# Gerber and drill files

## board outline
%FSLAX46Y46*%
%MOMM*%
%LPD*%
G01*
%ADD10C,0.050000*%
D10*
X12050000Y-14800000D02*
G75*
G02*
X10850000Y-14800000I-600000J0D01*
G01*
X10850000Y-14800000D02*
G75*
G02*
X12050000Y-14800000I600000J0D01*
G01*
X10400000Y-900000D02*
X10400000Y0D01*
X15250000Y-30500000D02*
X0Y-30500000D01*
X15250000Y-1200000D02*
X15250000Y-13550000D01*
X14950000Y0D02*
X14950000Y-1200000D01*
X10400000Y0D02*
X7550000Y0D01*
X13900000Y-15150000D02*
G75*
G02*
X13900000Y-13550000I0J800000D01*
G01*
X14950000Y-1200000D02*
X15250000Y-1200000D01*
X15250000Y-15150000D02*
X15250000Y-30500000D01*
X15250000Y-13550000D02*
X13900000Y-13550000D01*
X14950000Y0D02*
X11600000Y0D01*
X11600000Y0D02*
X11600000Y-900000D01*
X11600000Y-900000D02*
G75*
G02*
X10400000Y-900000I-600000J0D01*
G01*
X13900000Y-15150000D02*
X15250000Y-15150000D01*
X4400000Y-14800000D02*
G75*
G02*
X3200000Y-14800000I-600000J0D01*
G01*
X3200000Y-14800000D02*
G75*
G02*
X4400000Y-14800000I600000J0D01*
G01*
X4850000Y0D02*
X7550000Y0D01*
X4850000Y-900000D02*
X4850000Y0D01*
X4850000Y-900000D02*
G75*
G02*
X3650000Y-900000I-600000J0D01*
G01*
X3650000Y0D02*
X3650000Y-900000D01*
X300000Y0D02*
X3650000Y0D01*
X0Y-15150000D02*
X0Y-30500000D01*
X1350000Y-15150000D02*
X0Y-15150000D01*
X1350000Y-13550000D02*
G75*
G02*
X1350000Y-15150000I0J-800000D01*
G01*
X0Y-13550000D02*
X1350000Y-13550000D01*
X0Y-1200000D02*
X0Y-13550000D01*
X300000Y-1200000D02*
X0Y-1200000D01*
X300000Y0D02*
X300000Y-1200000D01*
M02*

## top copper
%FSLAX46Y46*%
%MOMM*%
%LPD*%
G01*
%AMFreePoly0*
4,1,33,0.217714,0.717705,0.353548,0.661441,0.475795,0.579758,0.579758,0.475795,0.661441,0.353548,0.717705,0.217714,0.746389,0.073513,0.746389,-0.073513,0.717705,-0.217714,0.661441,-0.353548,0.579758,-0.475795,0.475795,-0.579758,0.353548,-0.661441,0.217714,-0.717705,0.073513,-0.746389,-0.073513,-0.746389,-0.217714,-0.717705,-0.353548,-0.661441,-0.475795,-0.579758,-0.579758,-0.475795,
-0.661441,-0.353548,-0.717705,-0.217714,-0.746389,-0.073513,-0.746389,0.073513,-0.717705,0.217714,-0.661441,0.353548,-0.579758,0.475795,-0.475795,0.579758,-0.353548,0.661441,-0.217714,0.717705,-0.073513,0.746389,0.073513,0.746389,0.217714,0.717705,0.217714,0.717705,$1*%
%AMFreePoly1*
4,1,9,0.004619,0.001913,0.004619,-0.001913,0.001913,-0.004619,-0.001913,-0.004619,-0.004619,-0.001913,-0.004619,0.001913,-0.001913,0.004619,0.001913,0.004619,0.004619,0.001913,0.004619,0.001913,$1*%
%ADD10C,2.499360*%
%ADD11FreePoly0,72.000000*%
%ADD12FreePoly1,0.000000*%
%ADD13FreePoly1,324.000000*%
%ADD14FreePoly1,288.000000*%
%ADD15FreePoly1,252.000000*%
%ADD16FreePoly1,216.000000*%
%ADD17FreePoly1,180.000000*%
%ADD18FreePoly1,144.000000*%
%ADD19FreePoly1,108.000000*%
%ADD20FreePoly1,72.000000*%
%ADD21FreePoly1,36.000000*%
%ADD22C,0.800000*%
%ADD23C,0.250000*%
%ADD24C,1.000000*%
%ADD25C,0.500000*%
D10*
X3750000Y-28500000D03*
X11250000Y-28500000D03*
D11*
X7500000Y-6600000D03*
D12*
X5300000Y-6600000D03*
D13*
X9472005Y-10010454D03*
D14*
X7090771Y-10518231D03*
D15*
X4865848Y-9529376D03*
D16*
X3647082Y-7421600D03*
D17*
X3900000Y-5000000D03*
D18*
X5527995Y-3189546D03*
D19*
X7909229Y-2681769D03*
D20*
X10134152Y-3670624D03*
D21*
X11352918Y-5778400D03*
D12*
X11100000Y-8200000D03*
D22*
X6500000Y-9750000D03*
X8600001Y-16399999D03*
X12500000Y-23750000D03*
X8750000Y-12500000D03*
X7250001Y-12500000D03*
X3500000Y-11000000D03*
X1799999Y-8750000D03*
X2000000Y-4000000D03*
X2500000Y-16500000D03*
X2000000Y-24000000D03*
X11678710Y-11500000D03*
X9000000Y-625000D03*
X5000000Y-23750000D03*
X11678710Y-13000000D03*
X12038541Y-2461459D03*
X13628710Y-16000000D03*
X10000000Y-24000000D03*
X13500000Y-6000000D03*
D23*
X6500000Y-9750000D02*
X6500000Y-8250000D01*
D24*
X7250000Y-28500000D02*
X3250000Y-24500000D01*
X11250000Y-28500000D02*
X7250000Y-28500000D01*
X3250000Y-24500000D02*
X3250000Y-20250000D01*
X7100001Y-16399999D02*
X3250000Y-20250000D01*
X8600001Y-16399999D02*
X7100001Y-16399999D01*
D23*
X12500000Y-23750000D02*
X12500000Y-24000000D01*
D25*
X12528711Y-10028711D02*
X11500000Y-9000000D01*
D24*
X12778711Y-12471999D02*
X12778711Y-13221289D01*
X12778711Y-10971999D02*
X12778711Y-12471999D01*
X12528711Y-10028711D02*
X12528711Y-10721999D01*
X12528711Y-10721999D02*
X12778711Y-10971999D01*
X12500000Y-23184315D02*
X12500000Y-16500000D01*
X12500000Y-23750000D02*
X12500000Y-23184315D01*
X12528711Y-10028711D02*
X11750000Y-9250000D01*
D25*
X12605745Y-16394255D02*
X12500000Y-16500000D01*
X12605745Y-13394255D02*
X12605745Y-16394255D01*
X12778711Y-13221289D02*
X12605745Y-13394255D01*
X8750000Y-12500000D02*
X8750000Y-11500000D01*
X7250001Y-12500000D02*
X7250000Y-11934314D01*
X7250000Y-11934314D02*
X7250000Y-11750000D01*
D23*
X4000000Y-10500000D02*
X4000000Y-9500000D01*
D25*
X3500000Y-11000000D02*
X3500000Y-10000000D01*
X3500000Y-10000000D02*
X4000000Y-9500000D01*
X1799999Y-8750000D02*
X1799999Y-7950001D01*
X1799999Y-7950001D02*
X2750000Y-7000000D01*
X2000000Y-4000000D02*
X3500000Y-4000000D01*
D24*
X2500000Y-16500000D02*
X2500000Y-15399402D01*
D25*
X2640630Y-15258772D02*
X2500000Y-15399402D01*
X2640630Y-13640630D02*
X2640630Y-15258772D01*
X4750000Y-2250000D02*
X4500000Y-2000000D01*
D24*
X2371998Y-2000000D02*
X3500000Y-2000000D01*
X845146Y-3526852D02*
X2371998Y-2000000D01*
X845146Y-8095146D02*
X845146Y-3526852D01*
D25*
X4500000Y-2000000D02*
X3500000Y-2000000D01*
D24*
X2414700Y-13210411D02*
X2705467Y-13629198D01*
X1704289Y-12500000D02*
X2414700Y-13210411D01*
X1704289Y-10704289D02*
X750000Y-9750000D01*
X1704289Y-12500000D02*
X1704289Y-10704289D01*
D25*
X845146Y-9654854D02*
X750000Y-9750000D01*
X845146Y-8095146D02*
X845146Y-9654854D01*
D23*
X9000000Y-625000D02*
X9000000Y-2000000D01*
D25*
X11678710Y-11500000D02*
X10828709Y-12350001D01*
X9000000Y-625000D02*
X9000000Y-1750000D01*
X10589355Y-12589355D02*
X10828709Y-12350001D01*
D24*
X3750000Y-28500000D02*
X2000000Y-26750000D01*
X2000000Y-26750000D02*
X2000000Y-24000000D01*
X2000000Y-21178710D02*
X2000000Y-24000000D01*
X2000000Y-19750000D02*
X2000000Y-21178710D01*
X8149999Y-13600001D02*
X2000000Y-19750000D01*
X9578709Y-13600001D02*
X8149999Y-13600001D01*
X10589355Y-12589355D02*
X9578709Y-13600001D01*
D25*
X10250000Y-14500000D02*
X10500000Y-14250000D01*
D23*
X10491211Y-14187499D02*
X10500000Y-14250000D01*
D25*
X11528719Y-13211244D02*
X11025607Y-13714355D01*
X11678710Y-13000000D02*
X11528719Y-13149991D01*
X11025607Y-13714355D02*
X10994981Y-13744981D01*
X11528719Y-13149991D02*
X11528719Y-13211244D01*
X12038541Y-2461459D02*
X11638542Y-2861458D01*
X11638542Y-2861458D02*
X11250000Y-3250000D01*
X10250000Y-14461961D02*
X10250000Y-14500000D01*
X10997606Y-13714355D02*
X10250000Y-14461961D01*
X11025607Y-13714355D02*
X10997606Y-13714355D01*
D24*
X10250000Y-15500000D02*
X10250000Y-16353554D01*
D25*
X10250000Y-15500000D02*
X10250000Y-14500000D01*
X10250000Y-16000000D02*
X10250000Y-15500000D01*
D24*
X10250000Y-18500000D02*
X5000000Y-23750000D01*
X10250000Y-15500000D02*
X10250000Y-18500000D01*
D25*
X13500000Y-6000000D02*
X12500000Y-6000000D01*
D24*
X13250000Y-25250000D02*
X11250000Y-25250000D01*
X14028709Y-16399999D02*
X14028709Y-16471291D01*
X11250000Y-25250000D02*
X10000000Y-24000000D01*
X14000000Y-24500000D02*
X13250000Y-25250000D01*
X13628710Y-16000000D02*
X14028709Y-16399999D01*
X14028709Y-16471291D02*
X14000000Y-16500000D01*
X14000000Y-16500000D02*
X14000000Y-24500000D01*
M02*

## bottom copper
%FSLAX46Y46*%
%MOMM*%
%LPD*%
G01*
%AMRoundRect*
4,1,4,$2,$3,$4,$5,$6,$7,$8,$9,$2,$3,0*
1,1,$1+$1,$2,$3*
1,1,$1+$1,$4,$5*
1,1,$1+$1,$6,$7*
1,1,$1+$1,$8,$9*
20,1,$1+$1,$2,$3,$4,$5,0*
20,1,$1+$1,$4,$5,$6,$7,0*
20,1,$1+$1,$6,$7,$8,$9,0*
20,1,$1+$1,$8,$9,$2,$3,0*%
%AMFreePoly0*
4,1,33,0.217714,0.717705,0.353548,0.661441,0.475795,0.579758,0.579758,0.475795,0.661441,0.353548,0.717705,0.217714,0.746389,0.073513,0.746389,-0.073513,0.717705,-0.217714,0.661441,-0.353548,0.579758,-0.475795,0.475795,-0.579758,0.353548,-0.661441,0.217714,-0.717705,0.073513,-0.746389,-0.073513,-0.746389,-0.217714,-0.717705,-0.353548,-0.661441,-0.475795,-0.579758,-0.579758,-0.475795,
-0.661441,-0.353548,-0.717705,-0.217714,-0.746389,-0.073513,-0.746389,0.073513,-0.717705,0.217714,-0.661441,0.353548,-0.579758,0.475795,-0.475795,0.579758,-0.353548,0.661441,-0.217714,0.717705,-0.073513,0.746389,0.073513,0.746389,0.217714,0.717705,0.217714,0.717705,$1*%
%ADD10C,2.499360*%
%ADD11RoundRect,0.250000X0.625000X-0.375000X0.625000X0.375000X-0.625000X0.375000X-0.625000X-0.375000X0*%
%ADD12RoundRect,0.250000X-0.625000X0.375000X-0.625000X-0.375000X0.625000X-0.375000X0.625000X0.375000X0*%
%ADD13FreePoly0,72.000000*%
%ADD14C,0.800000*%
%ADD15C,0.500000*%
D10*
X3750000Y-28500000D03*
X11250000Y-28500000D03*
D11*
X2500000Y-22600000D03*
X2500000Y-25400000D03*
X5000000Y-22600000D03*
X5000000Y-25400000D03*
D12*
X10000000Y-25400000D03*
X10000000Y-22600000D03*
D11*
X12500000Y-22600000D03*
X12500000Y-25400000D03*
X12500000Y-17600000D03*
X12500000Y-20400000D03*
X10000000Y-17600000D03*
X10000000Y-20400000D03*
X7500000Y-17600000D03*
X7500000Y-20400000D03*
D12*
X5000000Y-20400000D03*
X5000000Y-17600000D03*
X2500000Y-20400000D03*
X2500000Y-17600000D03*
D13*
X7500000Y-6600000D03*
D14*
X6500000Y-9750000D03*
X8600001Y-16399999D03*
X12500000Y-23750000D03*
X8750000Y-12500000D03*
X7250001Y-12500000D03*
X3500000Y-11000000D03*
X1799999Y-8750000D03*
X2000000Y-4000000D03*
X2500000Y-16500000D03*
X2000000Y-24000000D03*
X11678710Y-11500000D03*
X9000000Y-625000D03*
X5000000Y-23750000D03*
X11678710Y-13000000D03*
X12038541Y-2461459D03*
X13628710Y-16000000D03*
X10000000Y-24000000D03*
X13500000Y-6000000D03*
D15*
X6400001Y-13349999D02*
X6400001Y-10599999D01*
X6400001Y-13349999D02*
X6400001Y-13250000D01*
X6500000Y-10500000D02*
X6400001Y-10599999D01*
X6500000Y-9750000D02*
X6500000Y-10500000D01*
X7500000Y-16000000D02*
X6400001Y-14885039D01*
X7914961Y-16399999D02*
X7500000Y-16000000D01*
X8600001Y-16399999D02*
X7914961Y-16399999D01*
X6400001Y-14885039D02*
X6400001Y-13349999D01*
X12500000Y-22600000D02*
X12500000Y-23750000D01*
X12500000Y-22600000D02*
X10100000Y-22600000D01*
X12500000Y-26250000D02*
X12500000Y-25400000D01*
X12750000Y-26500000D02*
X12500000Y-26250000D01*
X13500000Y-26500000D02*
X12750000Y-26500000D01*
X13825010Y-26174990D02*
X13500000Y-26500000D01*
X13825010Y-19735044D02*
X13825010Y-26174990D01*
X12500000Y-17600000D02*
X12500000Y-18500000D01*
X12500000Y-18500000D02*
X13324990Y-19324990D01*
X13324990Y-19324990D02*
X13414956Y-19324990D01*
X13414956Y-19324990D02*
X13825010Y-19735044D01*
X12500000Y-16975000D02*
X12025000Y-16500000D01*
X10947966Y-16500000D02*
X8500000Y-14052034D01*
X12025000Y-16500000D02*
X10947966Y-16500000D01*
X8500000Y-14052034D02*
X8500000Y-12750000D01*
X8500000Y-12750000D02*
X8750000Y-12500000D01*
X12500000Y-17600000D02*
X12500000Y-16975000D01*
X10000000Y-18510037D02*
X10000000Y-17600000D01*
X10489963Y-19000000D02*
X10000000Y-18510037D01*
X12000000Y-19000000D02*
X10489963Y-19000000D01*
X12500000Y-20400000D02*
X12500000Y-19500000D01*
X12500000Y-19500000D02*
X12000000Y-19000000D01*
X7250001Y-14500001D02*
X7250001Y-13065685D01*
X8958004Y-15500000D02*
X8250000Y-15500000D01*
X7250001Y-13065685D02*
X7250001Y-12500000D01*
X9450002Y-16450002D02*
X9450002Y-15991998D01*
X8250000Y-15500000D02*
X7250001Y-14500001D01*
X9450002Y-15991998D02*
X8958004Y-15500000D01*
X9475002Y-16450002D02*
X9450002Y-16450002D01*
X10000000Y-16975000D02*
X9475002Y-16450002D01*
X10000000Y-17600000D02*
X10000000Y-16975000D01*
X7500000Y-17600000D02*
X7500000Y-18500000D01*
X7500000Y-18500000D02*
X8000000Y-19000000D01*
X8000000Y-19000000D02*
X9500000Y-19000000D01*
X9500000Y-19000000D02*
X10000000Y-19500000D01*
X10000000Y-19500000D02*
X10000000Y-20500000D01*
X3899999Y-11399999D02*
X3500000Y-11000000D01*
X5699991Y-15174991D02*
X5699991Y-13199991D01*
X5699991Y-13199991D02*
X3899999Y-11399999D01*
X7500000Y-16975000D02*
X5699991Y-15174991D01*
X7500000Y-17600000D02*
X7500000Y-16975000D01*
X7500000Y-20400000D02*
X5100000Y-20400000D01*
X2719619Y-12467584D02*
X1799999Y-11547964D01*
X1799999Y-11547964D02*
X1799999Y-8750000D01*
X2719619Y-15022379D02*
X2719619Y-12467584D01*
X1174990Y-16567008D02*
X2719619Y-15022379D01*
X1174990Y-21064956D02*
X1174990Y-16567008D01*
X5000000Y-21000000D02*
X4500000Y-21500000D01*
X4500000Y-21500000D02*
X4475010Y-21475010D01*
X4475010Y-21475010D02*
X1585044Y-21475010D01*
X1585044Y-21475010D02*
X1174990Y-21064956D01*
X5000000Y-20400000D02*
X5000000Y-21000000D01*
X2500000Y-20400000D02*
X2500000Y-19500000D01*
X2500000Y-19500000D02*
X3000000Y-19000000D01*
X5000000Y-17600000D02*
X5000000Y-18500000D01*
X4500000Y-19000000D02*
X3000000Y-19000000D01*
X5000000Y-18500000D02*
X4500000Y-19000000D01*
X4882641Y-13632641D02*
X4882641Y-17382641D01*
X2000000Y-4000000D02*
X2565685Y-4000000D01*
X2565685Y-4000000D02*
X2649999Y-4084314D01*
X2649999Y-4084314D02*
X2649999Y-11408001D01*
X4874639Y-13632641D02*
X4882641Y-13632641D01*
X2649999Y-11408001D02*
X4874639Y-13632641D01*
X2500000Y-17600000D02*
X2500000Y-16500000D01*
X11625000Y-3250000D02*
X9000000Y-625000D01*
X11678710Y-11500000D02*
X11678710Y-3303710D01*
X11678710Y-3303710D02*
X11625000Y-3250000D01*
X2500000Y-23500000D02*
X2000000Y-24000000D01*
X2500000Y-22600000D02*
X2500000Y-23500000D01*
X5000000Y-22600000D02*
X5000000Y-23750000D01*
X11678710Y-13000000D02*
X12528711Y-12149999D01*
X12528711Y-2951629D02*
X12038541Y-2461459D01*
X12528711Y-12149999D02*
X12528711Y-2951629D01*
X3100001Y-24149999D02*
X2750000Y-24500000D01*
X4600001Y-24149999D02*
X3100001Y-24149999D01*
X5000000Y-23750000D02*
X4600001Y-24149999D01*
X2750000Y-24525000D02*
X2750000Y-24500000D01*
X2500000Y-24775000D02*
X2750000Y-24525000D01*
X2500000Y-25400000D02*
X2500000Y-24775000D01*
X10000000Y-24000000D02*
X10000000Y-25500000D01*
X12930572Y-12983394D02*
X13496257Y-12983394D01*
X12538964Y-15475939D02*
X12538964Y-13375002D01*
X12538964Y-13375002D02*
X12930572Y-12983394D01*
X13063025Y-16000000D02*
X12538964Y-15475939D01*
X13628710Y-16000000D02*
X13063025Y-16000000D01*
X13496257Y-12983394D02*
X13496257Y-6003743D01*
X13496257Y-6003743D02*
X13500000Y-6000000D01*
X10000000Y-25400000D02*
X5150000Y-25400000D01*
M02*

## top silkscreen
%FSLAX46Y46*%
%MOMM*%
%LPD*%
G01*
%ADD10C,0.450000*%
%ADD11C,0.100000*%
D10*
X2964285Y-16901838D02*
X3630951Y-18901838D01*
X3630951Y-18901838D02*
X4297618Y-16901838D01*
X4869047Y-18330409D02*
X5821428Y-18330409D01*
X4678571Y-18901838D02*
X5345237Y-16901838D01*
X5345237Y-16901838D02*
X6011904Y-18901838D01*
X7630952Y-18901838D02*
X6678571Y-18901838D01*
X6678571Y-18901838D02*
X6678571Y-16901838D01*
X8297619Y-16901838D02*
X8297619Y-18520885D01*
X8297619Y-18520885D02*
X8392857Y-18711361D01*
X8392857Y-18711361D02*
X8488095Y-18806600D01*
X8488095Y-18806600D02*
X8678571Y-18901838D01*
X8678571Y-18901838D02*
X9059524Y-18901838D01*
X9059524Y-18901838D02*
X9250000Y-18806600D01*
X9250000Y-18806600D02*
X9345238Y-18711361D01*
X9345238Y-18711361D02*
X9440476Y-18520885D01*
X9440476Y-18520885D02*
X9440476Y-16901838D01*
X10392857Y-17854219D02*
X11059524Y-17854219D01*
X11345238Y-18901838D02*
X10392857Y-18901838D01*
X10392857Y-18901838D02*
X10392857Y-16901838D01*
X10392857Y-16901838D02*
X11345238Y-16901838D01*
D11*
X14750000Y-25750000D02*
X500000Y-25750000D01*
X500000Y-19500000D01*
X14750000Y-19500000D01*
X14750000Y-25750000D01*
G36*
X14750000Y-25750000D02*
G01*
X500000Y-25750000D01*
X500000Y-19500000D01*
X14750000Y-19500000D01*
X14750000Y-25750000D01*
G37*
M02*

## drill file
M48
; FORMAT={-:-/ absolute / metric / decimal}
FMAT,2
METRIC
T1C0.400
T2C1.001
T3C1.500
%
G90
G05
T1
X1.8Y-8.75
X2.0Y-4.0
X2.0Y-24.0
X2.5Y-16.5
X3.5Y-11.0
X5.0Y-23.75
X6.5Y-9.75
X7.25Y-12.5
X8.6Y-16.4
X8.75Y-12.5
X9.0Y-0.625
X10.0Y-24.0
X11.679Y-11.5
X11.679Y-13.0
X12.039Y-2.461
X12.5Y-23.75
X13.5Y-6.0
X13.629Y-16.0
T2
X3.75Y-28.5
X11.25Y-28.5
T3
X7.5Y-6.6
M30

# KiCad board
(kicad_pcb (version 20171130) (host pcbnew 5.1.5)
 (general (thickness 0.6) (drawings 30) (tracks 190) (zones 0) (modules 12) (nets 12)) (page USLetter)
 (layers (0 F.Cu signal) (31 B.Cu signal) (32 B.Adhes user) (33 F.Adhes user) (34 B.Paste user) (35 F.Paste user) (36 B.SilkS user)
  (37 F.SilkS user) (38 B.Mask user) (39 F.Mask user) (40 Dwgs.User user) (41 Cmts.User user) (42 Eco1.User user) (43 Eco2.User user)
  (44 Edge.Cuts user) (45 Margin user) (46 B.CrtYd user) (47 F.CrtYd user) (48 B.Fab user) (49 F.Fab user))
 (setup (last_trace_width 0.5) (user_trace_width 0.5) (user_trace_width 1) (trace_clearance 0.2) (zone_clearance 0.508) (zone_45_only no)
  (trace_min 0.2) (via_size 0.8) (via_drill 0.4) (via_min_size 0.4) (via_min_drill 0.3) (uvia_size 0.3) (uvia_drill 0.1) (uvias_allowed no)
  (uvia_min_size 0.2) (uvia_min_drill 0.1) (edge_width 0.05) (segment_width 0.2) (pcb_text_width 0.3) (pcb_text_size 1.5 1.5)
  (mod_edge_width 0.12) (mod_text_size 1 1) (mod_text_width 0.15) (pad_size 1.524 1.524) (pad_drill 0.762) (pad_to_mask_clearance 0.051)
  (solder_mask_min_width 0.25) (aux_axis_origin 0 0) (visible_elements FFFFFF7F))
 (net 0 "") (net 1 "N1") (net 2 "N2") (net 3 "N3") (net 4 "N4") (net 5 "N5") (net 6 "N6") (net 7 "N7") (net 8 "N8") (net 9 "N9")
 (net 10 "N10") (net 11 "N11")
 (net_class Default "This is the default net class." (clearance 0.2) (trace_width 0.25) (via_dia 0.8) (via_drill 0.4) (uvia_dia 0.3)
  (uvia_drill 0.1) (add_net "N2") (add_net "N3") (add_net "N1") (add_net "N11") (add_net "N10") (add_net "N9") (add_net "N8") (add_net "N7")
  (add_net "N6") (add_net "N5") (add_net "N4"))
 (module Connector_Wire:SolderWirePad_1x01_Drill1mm (layer F.Cu) (at 3.75 28.5)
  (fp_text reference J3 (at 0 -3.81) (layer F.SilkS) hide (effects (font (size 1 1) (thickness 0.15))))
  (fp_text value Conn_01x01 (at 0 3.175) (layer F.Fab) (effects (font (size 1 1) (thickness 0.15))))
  (pad 1 thru_hole circle (at 0 0) (size 2.49936 2.49936) (drill 1.00076) (layers *.Cu *.Mask) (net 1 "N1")))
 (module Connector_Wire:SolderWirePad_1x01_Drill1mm (layer F.Cu) (at 11.25 28.5)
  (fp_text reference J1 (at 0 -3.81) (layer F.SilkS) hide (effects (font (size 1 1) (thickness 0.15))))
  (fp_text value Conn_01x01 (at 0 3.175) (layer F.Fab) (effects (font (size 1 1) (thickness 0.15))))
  (pad 1 thru_hole circle (at 0 0) (size 2.49936 2.49936) (drill 1.00076) (layers *.Cu *.Mask) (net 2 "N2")))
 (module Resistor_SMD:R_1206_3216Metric (layer B.Cu) (at 2.5 24 90)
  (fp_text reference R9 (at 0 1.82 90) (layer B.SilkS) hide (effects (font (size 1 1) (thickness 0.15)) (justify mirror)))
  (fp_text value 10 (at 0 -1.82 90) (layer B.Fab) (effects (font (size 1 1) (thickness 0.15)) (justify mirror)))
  (pad 2 smd roundrect (at 1.4 0 90) (size 1.25 1.75) (layers B.Cu B.Paste B.Mask) (roundrect_rratio 0.2) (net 1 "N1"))
  (pad 1 smd roundrect (at -1.4 0 90) (size 1.25 1.75) (layers B.Cu B.Paste B.Mask) (roundrect_rratio 0.2) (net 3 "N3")))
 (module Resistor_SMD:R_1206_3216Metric (layer B.Cu) (at 5 24 90)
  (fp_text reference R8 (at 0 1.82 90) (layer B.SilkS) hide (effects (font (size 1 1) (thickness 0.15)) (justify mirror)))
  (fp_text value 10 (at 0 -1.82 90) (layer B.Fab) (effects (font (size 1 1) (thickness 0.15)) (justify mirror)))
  (pad 2 smd roundrect (at 1.4 0 90) (size 1.25 1.75) (layers B.Cu B.Paste B.Mask) (roundrect_rratio 0.2) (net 3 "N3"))
  (pad 1 smd roundrect (at -1.4 0 90) (size 1.25 1.75) (layers B.Cu B.Paste B.Mask) (roundrect_rratio 0.2) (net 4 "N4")))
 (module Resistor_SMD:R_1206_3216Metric (layer B.Cu) (at 10 24 270)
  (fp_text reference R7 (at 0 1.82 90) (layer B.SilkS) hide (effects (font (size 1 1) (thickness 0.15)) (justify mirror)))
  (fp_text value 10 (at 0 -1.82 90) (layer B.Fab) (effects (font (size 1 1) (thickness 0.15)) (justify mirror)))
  (pad 2 smd roundrect (at 1.4 0 270) (size 1.25 1.75) (layers B.Cu B.Paste B.Mask) (roundrect_rratio 0.2) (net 4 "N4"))
  (pad 1 smd roundrect (at -1.4 0 270) (size 1.25 1.75) (layers B.Cu B.Paste B.Mask) (roundrect_rratio 0.2) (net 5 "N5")))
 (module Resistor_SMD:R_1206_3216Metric (layer B.Cu) (at 12.5 24 90)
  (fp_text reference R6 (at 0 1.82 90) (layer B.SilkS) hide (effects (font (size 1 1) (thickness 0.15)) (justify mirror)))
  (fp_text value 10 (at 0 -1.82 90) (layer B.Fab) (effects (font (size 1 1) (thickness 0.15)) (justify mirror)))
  (pad 2 smd roundrect (at 1.4 0 90) (size 1.25 1.75) (layers B.Cu B.Paste B.Mask) (roundrect_rratio 0.2) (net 5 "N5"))
  (pad 1 smd roundrect (at -1.4 0 90) (size 1.25 1.75) (layers B.Cu B.Paste B.Mask) (roundrect_rratio 0.2) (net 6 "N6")))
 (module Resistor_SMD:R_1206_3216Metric (layer B.Cu) (at 12.5 19 90)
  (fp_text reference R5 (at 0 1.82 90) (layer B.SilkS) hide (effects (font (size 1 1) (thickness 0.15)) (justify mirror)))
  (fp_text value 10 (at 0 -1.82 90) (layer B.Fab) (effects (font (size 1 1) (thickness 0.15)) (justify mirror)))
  (pad 2 smd roundrect (at 1.4 0 90) (size 1.25 1.75) (layers B.Cu B.Paste B.Mask) (roundrect_rratio 0.2) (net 6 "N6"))
  (pad 1 smd roundrect (at -1.4 0 90) (size 1.25 1.75) (layers B.Cu B.Paste B.Mask) (roundrect_rratio 0.2) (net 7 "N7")))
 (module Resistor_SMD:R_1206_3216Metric (layer B.Cu) (at 10 19 90)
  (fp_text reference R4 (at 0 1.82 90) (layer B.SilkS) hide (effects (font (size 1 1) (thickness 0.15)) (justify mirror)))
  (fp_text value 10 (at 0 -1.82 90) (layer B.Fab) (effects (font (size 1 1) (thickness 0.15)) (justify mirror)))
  (pad 2 smd roundrect (at 1.4 0 90) (size 1.25 1.75) (layers B.Cu B.Paste B.Mask) (roundrect_rratio 0.2) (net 7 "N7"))
  (pad 1 smd roundrect (at -1.4 0 90) (size 1.25 1.75) (layers B.Cu B.Paste B.Mask) (roundrect_rratio 0.2) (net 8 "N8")))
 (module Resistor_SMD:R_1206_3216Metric (layer B.Cu) (at 7.5 19 90)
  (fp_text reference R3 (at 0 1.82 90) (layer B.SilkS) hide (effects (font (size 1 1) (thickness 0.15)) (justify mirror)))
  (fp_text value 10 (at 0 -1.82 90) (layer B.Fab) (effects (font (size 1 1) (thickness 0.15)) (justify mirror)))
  (pad 2 smd roundrect (at 1.4 0 90) (size 1.25 1.75) (layers B.Cu B.Paste B.Mask) (roundrect_rratio 0.2) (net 8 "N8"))
  (pad 1 smd roundrect (at -1.4 0 90) (size 1.25 1.75) (layers B.Cu B.Paste B.Mask) (roundrect_rratio 0.2) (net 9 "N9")))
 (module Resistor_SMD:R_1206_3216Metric (layer B.Cu) (at 5 19 270)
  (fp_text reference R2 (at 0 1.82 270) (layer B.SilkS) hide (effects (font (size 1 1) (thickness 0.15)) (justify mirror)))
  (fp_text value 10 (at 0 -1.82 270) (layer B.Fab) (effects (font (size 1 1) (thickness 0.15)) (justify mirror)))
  (pad 2 smd roundrect (at 1.4 0 270) (size 1.25 1.75) (layers B.Cu B.Paste B.Mask) (roundrect_rratio 0.2) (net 9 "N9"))
  (pad 1 smd roundrect (at -1.4 0 270) (size 1.25 1.75) (layers B.Cu B.Paste B.Mask) (roundrect_rratio 0.2) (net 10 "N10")))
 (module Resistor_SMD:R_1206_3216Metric (layer B.Cu) (at 2.5 19 270)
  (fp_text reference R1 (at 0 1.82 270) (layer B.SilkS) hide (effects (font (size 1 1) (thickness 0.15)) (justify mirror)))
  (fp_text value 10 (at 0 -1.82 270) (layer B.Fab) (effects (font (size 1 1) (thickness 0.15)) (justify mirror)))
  (pad 2 smd roundrect (at 1.4 0 270) (size 1.25 1.75) (layers B.Cu B.Paste B.Mask) (roundrect_rratio 0.2) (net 10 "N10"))
  (pad 1 smd roundrect (at -1.4 0 270) (size 1.25 1.75) (layers B.Cu B.Paste B.Mask) (roundrect_rratio 0.2) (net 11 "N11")))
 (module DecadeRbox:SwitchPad (layer F.Cu) (at 7.5 6.6)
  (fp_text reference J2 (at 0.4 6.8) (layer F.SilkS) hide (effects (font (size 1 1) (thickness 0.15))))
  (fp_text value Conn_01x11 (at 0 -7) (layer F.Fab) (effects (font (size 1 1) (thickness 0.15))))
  (pad "" np_thru_hole custom (at 0 0 72) (size 1.5 1.5) (drill 1.5) (layers *.Cu *.Mask) (zone_connect 0)
   (options (clearance outline) (anchor circle)) (primitives))
  (pad 1 smd custom (at -2.2 0) (size 0.01 0.01) (layers F.Cu F.Mask) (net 2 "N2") (zone_connect 0)
   (options (clearance outline) (anchor circle)) (primitives))
  (pad 8 smd custom (at 1.972005 3.410454 324) (size 0.01 0.01) (layers F.Cu F.Mask) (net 5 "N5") (zone_connect 0)
   (options (clearance outline) (anchor circle)) (primitives))
  (pad 7 smd custom (at -0.409229 3.918231 288) (size 0.01 0.01) (layers F.Cu F.Mask) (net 6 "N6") (zone_connect 0)
   (options (clearance outline) (anchor circle)) (primitives))
  (pad 6 smd custom (at -2.634152 2.929376 252) (size 0.01 0.01) (layers F.Cu F.Mask) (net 7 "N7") (zone_connect 0)
   (options (clearance outline) (anchor circle)) (primitives))
  (pad 5 smd custom (at -3.852918 0.8216 216) (size 0.01 0.01) (layers F.Cu F.Mask) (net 8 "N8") (zone_connect 0)
   (options (clearance outline) (anchor circle)) (primitives))
  (pad 4 smd custom (at -3.6 -1.6 180) (size 0.01 0.01) (layers F.Cu F.Mask) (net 9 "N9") (zone_connect 0)
   (options (clearance outline) (anchor circle)) (primitives))
  (pad 3 smd custom (at -1.972005 -3.410454 144) (size 0.01 0.01) (layers F.Cu F.Mask) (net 10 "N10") (zone_connect 0)
   (options (clearance outline) (anchor circle)) (primitives))
  (pad 2 smd custom (at 0.409229 -3.918231 108) (size 0.01 0.01) (layers F.Cu F.Mask) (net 11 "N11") (zone_connect 0)
   (options (clearance outline) (anchor circle)) (primitives))
  (pad 11 smd custom (at 2.634152 -2.929376 72) (size 0.01 0.01) (layers F.Cu F.Mask) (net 1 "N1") (zone_connect 0)
   (options (clearance outline) (anchor circle)) (primitives))
  (pad 10 smd custom (at 3.852918 -0.8216 36) (size 0.01 0.01) (layers F.Cu F.Mask) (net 3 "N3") (zone_connect 0)
   (options (clearance outline) (anchor circle)) (primitives))
  (pad 9 smd custom (at 3.6 1.6) (size 0.01 0.01) (layers F.Cu F.Mask) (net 4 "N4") (zone_connect 0)
   (options (clearance outline) (anchor circle)) (primitives)))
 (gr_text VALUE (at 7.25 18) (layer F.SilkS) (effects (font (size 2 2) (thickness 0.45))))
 (gr_poly (pts (xy 14.75 25.75) (xy 0.5 25.75) (xy 0.5 19.5) (xy 14.75 19.5)) (layer F.SilkS) (width 0.1))
 (gr_circle (center 11.45 14.8) (end 10.85 14.8) (layer Edge.Cuts) (width 0.05))
 (gr_line (start 10.4 0.9) (end 10.4 0) (layer Edge.Cuts) (width 0.05))
 (gr_line (start 15.25 30.5) (end 0 30.5) (layer Edge.Cuts) (width 0.05))
 (gr_line (start 15.25 1.2) (end 15.25 13.55) (layer Edge.Cuts) (width 0.05))
 (gr_line (start 14.95 0) (end 14.95 1.2) (layer Edge.Cuts) (width 0.05))
 (gr_line (start 10.4 0) (end 7.55 0) (layer Edge.Cuts) (width 0.05))
 (gr_arc (start 13.9 14.35) (end 13.9 15.15) (angle 180) (layer Edge.Cuts) (width 0.05))
 (gr_line (start 14.95 1.2) (end 15.25 1.2) (layer Edge.Cuts) (width 0.05))
 (gr_line (start 15.25 15.15) (end 15.25 30.5) (layer Edge.Cuts) (width 0.05))
 (gr_line (start 15.25 13.55) (end 13.9 13.55) (layer Edge.Cuts) (width 0.05))
 (gr_line (start 14.95 0) (end 11.6 0) (layer Edge.Cuts) (width 0.05))
 (gr_line (start 11.6 0) (end 11.6 0.9) (layer Edge.Cuts) (width 0.05))
 (gr_arc (start 11 0.9) (end 11.6 0.9) (angle 180) (layer Edge.Cuts) (width 0.05))
 (gr_line (start 13.9 15.15) (end 15.25 15.15) (layer Edge.Cuts) (width 0.05))
 (gr_circle (center 3.8 14.8) (end 4.4 14.8) (layer Edge.Cuts) (width 0.05))
 (gr_line (start 4.85 0) (end 7.55 0) (layer Edge.Cuts) (width 0.05))
 (gr_line (start 4.85 0.9) (end 4.85 0) (layer Edge.Cuts) (width 0.05))
 (gr_arc (start 4.25 0.9) (end 3.65 0.9) (angle -180) (layer Edge.Cuts) (width 0.05))
 (gr_line (start 3.65 0) (end 3.65 0.9) (layer Edge.Cuts) (width 0.05))
 (gr_line (start 0.3 0) (end 3.65 0) (layer Edge.Cuts) (width 0.05))
 (gr_line (start 0 15.15) (end 0 30.5) (layer Edge.Cuts) (width 0.05))
 (gr_line (start 1.35 15.15) (end 0 15.15) (layer Edge.Cuts) (width 0.05))
 (gr_arc (start 1.35 14.35) (end 1.35 15.15) (angle -180) (layer Edge.Cuts) (width 0.05))
 (gr_line (start 0 13.55) (end 1.35 13.55) (layer Edge.Cuts) (width 0.05))
 (gr_line (start 0 1.2) (end 0 13.55) (layer Edge.Cuts) (width 0.05))
 (gr_line (start 0.3 1.2) (end 0 1.2) (layer Edge.Cuts) (width 0.05))
 (gr_line (start 0.3 0) (end 0.3 1.2) (layer Edge.Cuts) (width 0.05))
 (via (at 6.5 9.75) (size 0.8) (drill 0.4) (layers F.Cu B.Cu) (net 2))
 (segment (start 6.5 9.75) (end 6.5 8.25) (width 0.25) (layer F.Cu) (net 2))
 (segment (start 6.400001 13.349999) (end 6.400001 10.599999) (width 0.5) (layer B.Cu) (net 2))
 (segment (start 6.400001 13.349999) (end 6.400001 13.25) (width 0.5) (layer B.Cu) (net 2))
 (segment (start 6.5 10.5) (end 6.400001 10.599999) (width 0.5) (layer B.Cu) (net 2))
 (segment (start 6.5 9.75) (end 6.5 10.5) (width 0.5) (layer B.Cu) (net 2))
 (segment (start 7.5 16) (end 6.400001 14.885039) (width 0.5) (layer B.Cu) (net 2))
 (segment (start 7.914961 16.399999) (end 7.5 16) (width 0.5) (layer B.Cu) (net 2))
 (segment (start 8.600001 16.399999) (end 7.914961 16.399999) (width 0.5) (layer B.Cu) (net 2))
 (via (at 8.600001 16.399999) (size 0.8) (drill 0.4) (layers F.Cu B.Cu) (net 2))
 (segment (start 6.400001 14.885039) (end 6.400001 13.349999) (width 0.5) (layer B.Cu) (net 2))
 (segment (start 7.25 28.5) (end 3.25 24.5) (width 1) (layer F.Cu) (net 2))
 (segment (start 11.25 28.5) (end 7.25 28.5) (width 1) (layer F.Cu) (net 2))
 (segment (start 3.25 24.5) (end 3.25 20.25) (width 1) (layer F.Cu) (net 2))
 (segment (start 7.100001 16.399999) (end 3.25 20.25) (width 1) (layer F.Cu) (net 2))
 (segment (start 8.600001 16.399999) (end 7.100001 16.399999) (width 1) (layer F.Cu) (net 2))
 (via (at 12.5 23.75) (size 0.8) (drill 0.4) (layers F.Cu B.Cu) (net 5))
 (segment (start 12.5 22.6) (end 12.5 23.75) (width 0.5) (layer B.Cu) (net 5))
 (segment (start 12.5 23.75) (end 12.5 24) (width 0.25) (layer F.Cu) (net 5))
 (segment (start 12.528711 10.028711) (end 11.5 9) (width 0.5) (layer F.Cu) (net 5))
 (segment (start 12.5 22.6) (end 10.1 22.6) (width 0.5) (layer B.Cu) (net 5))
 (segment (start 12.778711 12.471999) (end 12.778711 13.221289) (width 1) (layer F.Cu) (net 5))
 (segment (start 12.778711 10.971999) (end 12.778711 12.471999) (width 1) (layer F.Cu) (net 5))
 (segment (start 12.528711 10.028711) (end 12.528711 10.721999) (width 1) (layer F.Cu) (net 5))
 (segment (start 12.528711 10.721999) (end 12.778711 10.971999) (width 1) (layer F.Cu) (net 5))
 (segment (start 12.5 23.184315) (end 12.5 16.5) (width 1) (layer F.Cu) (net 5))
 (segment (start 12.5 23.75) (end 12.5 23.184315) (width 1) (layer F.Cu) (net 5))
 (segment (start 12.528711 10.028711) (end 11.75 9.25) (width 1) (layer F.Cu) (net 5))
 (segment (start 12.605745 16.394255) (end 12.5 16.5) (width 0.5) (layer F.Cu) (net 5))
 (segment (start 12.605745 13.394255) (end 12.605745 16.394255) (width 0.5) (layer F.Cu) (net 5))
 (segment (start 12.778711 13.221289) (end 12.605745 13.394255) (width 0.5) (layer F.Cu) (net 5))
 (segment (start 12.5 26.25) (end 12.5 25.4) (width 0.5) (layer B.Cu) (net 6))
 (segment (start 12.75 26.5) (end 12.5 26.25) (width 0.5) (layer B.Cu) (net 6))
 (segment (start 13.5 26.5) (end 12.75 26.5) (width 0.5) (layer B.Cu) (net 6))
 (segment (start 13.82501 26.17499) (end 13.5 26.5) (width 0.5) (layer B.Cu) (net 6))
 (segment (start 13.82501 19.735044) (end 13.82501 26.17499) (width 0.5) (layer B.Cu) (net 6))
 (segment (start 12.5 17.6) (end 12.5 18.5) (width 0.5) (layer B.Cu) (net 6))
 (segment (start 12.5 18.5) (end 13.32499 19.32499) (width 0.5) (layer B.Cu) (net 6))
 (segment (start 13.32499 19.32499) (end 13.414956 19.32499) (width 0.5) (layer B.Cu) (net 6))
 (segment (start 13.414956 19.32499) (end 13.82501 19.735044) (width 0.5) (layer B.Cu) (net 6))
 (segment (start 12.5 16.975) (end 12.025 16.5) (width 0.5) (layer B.Cu) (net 6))
 (segment (start 10.947966 16.5) (end 8.5 14.052034) (width 0.5) (layer B.Cu) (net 6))
 (segment (start 12.025 16.5) (end 10.947966 16.5) (width 0.5) (layer B.Cu) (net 6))
 (segment (start 8.5 14.052034) (end 8.5 12.75) (width 0.5) (layer B.Cu) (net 6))
 (via (at 8.75 12.5) (size 0.8) (drill 0.4) (layers F.Cu B.Cu) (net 6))
 (segment (start 8.5 12.75) (end 8.75 12.5) (width 0.5) (layer B.Cu) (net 6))
 (segment (start 8.75 12.5) (end 8.75 11.5) (width 0.5) (layer F.Cu) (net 6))
 (segment (start 12.5 17.6) (end 12.5 16.975) (width 0.5) (layer B.Cu) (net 6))
 (segment (start 10 18.510037) (end 10 17.6) (width 0.5) (layer B.Cu) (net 7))
 (segment (start 10.489963 19) (end 10 18.510037) (width 0.5) (layer B.Cu) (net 7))
 (segment (start 12 19) (end 10.489963 19) (width 0.5) (layer B.Cu) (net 7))
 (segment (start 12.5 20.4) (end 12.5 19.5) (width 0.5) (layer B.Cu) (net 7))
 (segment (start 12.5 19.5) (end 12 19) (width 0.5) (layer B.Cu) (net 7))
 (via (at 7.250001 12.5) (size 0.8) (drill 0.4) (layers F.Cu B.Cu) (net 7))
 (segment (start 7.250001 12.5) (end 7.25 11.934314) (width 0.5) (layer F.Cu) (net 7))
 (segment (start 7.25 11.934314) (end 7.25 11.75) (width 0.5) (layer F.Cu) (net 7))
 (segment (start 7.250001 14.500001) (end 7.250001 13.065685) (width 0.5) (layer B.Cu) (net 7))
 (segment (start 8.958004 15.5) (end 8.25 15.5) (width 0.5) (layer B.Cu) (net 7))
 (segment (start 7.250001 13.065685) (end 7.250001 12.5) (width 0.5) (layer B.Cu) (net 7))
 (segment (start 9.450002 16.450002) (end 9.450002 15.991998) (width 0.5) (layer B.Cu) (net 7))
 (segment (start 8.25 15.5) (end 7.250001 14.500001) (width 0.5) (layer B.Cu) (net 7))
 (segment (start 9.450002 15.991998) (end 8.958004 15.5) (width 0.5) (layer B.Cu) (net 7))
 (segment (start 9.475002 16.450002) (end 9.450002 16.450002) (width 0.5) (layer B.Cu) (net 7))
 (segment (start 10 16.975) (end 9.475002 16.450002) (width 0.5) (layer B.Cu) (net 7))
 (segment (start 10 17.6) (end 10 16.975) (width 0.5) (layer B.Cu) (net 7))
 (via (at 3.5 11) (size 0.8) (drill 0.4) (layers F.Cu B.Cu) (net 8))
 (segment (start 4 10.5) (end 4 9.5) (width 0.25) (layer F.Cu) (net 8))
 (segment (start 7.5 17.6) (end 7.5 18.5) (width 0.5) (layer B.Cu) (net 8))
 (segment (start 7.5 18.5) (end 8 19) (width 0.5) (layer B.Cu) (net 8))
 (segment (start 8 19) (end 9.5 19) (width 0.5) (layer B.Cu) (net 8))
 (segment (start 9.5 19) (end 10 19.5) (width 0.5) (layer B.Cu) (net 8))
 (segment (start 10 19.5) (end 10 20.5) (width 0.5) (layer B.Cu) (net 8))
 (segment (start 3.899999 11.399999) (end 3.5 11) (width 0.5) (layer B.Cu) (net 8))
 (segment (start 5.699991 15.174991) (end 5.699991 13.199991) (width 0.5) (layer B.Cu) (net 8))
 (segment (start 5.699991 13.199991) (end 3.899999 11.399999) (width 0.5) (layer B.Cu) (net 8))
 (segment (start 7.5 16.975) (end 5.699991 15.174991) (width 0.5) (layer B.Cu) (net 8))
 (segment (start 7.5 17.6) (end 7.5 16.975) (width 0.5) (layer B.Cu) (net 8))
 (segment (start 3.5 11) (end 3.5 10) (width 0.5) (layer F.Cu) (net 8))
 (segment (start 3.5 10) (end 4 9.5) (width 0.5) (layer F.Cu) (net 8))
 (segment (start 7.5 20.4) (end 5.1 20.4) (width 0.5) (layer B.Cu) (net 9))
 (via (at 1.799999 8.75) (size 0.8) (drill 0.4) (layers F.Cu B.Cu) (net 9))
 (segment (start 1.799999 8.75) (end 1.799999 7.950001) (width 0.5) (layer F.Cu) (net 9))
 (segment (start 1.799999 7.950001) (end 2.75 7) (width 0.5) (layer F.Cu) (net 9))
 (segment (start 2.719619 12.467584) (end 1.799999 11.547964) (width 0.5) (layer B.Cu) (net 9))
 (segment (start 1.799999 11.547964) (end 1.799999 8.75) (width 0.5) (layer B.Cu) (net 9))
 (segment (start 2.719619 15.022379) (end 2.719619 12.467584) (width 0.5) (layer B.Cu) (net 9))
 (segment (start 1.17499 16.567008) (end 2.719619 15.022379) (width 0.5) (layer B.Cu) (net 9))
 (segment (start 1.17499 21.064956) (end 1.17499 16.567008) (width 0.5) (layer B.Cu) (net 9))
 (segment (start 5 21) (end 4.5 21.5) (width 0.5) (layer B.Cu) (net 9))
 (segment (start 4.5 21.5) (end 4.47501 21.47501) (width 0.5) (layer B.Cu) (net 9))
 (segment (start 4.47501 21.47501) (end 1.585044 21.47501) (width 0.5) (layer B.Cu) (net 9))
 (segment (start 1.585044 21.47501) (end 1.17499 21.064956) (width 0.5) (layer B.Cu) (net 9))
 (segment (start 5 20.4) (end 5 21) (width 0.5) (layer B.Cu) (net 9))
 (via (at 2 4) (size 0.8) (drill 0.4) (layers F.Cu B.Cu) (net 10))
 (segment (start 2.5 20.4) (end 2.5 19.5) (width 0.5) (layer B.Cu) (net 10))
 (segment (start 2.5 19.5) (end 3 19) (width 0.5) (layer B.Cu) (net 10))
 (segment (start 5 17.6) (end 5 18.5) (width 0.5) (layer B.Cu) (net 10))
 (segment (start 4.5 19) (end 3 19) (width 0.5) (layer B.Cu) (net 10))
 (segment (start 5 18.5) (end 4.5 19) (width 0.5) (layer B.Cu) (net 10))
 (segment (start 2 4) (end 3.5 4) (width 0.5) (layer F.Cu) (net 10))
 (segment (start 4.882641 13.632641) (end 4.882641 17.382641) (width 0.5) (layer B.Cu) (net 10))
 (segment (start 2 4) (end 2.565685 4) (width 0.5) (layer B.Cu) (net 10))
 (segment (start 2.565685 4) (end 2.649999 4.084314) (width 0.5) (layer B.Cu) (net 10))
 (segment (start 2.649999 4.084314) (end 2.649999 11.408001) (width 0.5) (layer B.Cu) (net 10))
 (segment (start 4.874639 13.632641) (end 4.882641 13.632641) (width 0.5) (layer B.Cu) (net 10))
 (segment (start 2.649999 11.408001) (end 4.874639 13.632641) (width 0.5) (layer B.Cu) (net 10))
 (via (at 2.5 16.5) (size 0.8) (drill 0.4) (layers F.Cu B.Cu) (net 11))
 (segment (start 2.5 17.6) (end 2.5 16.5) (width 0.5) (layer B.Cu) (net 11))
 (segment (start 2.5 16.5) (end 2.5 15.399402) (width 1) (layer F.Cu) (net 11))
 (segment (start 2.64063 15.258772) (end 2.5 15.399402) (width 0.5) (layer F.Cu) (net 11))
 (segment (start 2.64063 13.64063) (end 2.64063 15.258772) (width 0.5) (layer F.Cu) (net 11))
 (segment (start 4.75 2.25) (end 4.5 2) (width 0.5) (layer F.Cu) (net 11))
 (segment (start 2.371998 2) (end 3.5 2) (width 1) (layer F.Cu) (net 11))
 (segment (start 0.845146 3.526852) (end 2.371998 2) (width 1) (layer F.Cu) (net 11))
 (segment (start 0.845146 8.095146) (end 0.845146 3.526852) (width 1) (layer F.Cu) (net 11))
 (segment (start 4.5 2) (end 3.5 2) (width 0.5) (layer F.Cu) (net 11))
 (segment (start 2.4147 13.210411) (end 2.705467 13.629198) (width 1) (layer F.Cu) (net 11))
 (segment (start 1.704289 12.5) (end 2.4147 13.210411) (width 1) (layer F.Cu) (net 11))
 (segment (start 1.704289 10.704289) (end 0.75 9.75) (width 1) (layer F.Cu) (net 11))
 (segment (start 1.704289 12.5) (end 1.704289 10.704289) (width 1) (layer F.Cu) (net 11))
 (segment (start 0.845146 9.654854) (end 0.75 9.75) (width 0.5) (layer F.Cu) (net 11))
 (segment (start 0.845146 8.095146) (end 0.845146 9.654854) (width 0.5) (layer F.Cu) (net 11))
 (via (at 2 24) (size 0.8) (drill 0.4) (layers F.Cu B.Cu) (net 1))
 (via (at 11.67871 11.5) (size 0.8) (drill 0.4) (layers F.Cu B.Cu) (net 1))
 (via (at 9 0.625) (size 0.8) (drill 0.4) (layers F.Cu B.Cu) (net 1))
 (segment (start 9 0.625) (end 9 2) (width 0.25) (layer F.Cu) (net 1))
 (segment (start 11.67871 11.5) (end 10.828709 12.350001) (width 0.5) (layer F.Cu) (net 1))
 (segment (start 11.625 3.25) (end 9 0.625) (width 0.5) (layer B.Cu) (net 1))
 (segment (start 11.67871 11.5) (end 11.67871 3.30371) (width 0.5) (layer B.Cu) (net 1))
 (segment (start 11.67871 3.30371) (end 11.625 3.25) (width 0.5) (layer B.Cu) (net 1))
 (segment (start 9 0.625) (end 9 1.75) (width 0.5) (layer F.Cu) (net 1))
 (segment (start 2.5 23.5) (end 2 24) (width 0.5) (layer B.Cu) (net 1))
 (segment (start 2.5 22.6) (end 2.5 23.5) (width 0.5) (layer B.Cu) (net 1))
 (segment (start 10.589355 12.589355) (end 10.828709 12.350001) (width 0.5) (layer F.Cu) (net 1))
 (segment (start 3.75 28.5) (end 2 26.75) (width 1) (layer F.Cu) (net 1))
 (segment (start 2 26.75) (end 2 24) (width 1) (layer F.Cu) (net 1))
 (segment (start 2 21.17871) (end 2 24) (width 1) (layer F.Cu) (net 1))
 (segment (start 2 19.75) (end 2 21.17871) (width 1) (layer F.Cu) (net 1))
 (segment (start 8.149999 13.600001) (end 2 19.75) (width 1) (layer F.Cu) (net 1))
 (segment (start 9.578709 13.600001) (end 8.149999 13.600001) (width 1) (layer F.Cu) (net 1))
 (segment (start 10.589355 12.589355) (end 9.578709 13.600001) (width 1) (layer F.Cu) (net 1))
 (via (at 5 23.75) (size 0.8) (drill 0.4) (layers F.Cu B.Cu) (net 3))
 (segment (start 5 22.6) (end 5 23.75) (width 0.5) (layer B.Cu) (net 3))
 (via (at 11.67871 13) (size 0.8) (drill 0.4) (layers F.Cu B.Cu) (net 3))
 (segment (start 10.25 14.5) (end 10.5 14.25) (width 0.5) (layer F.Cu) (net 3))
 (segment (start 10.491211 14.187499) (end 10.5 14.25) (width 0.25) (layer F.Cu) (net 3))
 (segment (start 11.528719 13.211244) (end 11.025607 13.714355) (width 0.5) (layer F.Cu) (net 3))
 (segment (start 11.67871 13) (end 11.528719 13.149991) (width 0.5) (layer F.Cu) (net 3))
 (segment (start 11.025607 13.714355) (end 10.994981 13.744981) (width 0.5) (layer F.Cu) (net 3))
 (segment (start 11.528719 13.149991) (end 11.528719 13.211244) (width 0.5) (layer F.Cu) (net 3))
 (via (at 12.038541 2.461459) (size 0.8) (drill 0.4) (layers F.Cu B.Cu) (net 3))
 (segment (start 11.67871 13) (end 12.528711 12.149999) (width 0.5) (layer B.Cu) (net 3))
 (segment (start 12.528711 2.951629) (end 12.038541 2.461459) (width 0.5) (layer B.Cu) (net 3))
 (segment (start 12.528711 12.149999) (end 12.528711 2.951629) (width 0.5) (layer B.Cu) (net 3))
 (segment (start 12.038541 2.461459) (end 11.638542 2.861458) (width 0.5) (layer F.Cu) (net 3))
 (segment (start 11.638542 2.861458) (end 11.25 3.25) (width 0.5) (layer F.Cu) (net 3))
 (segment (start 3.100001 24.149999) (end 2.75 24.5) (width 0.5) (layer B.Cu) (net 3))
 (segment (start 4.600001 24.149999) (end 3.100001 24.149999) (width 0.5) (layer B.Cu) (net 3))
 (segment (start 5 23.75) (end 4.600001 24.149999) (width 0.5) (layer B.Cu) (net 3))
 (segment (start 2.75 24.525) (end 2.75 24.5) (width 0.5) (layer B.Cu) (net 3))
 (segment (start 2.5 24.775) (end 2.75 24.525) (width 0.5) (layer B.Cu) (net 3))
 (segment (start 2.5 25.4) (end 2.5 24.775) (width 0.5) (layer B.Cu) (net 3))
 (segment (start 10.25 14.461961) (end 10.25 14.5) (width 0.5) (layer F.Cu) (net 3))
 (segment (start 10.997606 13.714355) (end 10.25 14.461961) (width 0.5) (layer F.Cu) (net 3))
 (segment (start 11.025607 13.714355) (end 10.997606 13.714355) (width 0.5) (layer F.Cu) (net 3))
 (segment (start 10.25 15.5) (end 10.25 16.353554) (width 1) (layer F.Cu) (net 3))
 (segment (start 10.25 15.5) (end 10.25 14.5) (width 0.5) (layer F.Cu) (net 3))
 (segment (start 10.25 16) (end 10.25 15.5) (width 0.5) (layer F.Cu) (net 3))
 (segment (start 10.25 18.5) (end 5 23.75) (width 1) (layer F.Cu) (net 3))
 (segment (start 10.25 15.5) (end 10.25 18.5) (width 1) (layer F.Cu) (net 3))
 (via (at 13.62871 16) (size 0.8) (drill 0.4) (layers F.Cu B.Cu) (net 4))
 (via (at 10 24) (size 0.8) (drill 0.4) (layers F.Cu B.Cu) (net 4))
 (segment (start 10 24) (end 10 25.5) (width 0.5) (layer B.Cu) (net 4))
 (segment (start 12.930572 12.983394) (end 13.496257 12.983394) (width 0.5) (layer B.Cu) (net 4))
 (segment (start 12.538964 15.475939) (end 12.538964 13.375002) (width 0.5) (layer B.Cu) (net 4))
 (segment (start 12.538964 13.375002) (end 12.930572 12.983394) (width 0.5) (layer B.Cu) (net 4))
 (segment (start 13.063025 16) (end 12.538964 15.475939) (width 0.5) (layer B.Cu) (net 4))
 (segment (start 13.62871 16) (end 13.063025 16) (width 0.5) (layer B.Cu) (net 4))
 (segment (start 13.496257 12.983394) (end 13.496257 6.003743) (width 0.5) (layer B.Cu) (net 4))
 (via (at 13.5 6) (size 0.8) (drill 0.4) (layers F.Cu B.Cu) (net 4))
 (segment (start 13.496257 6.003743) (end 13.5 6) (width 0.5) (layer B.Cu) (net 4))
 (segment (start 13.5 6) (end 12.5 6) (width 0.5) (layer F.Cu) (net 4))
 (segment (start 10 25.4) (end 5.15 25.4) (width 0.5) (layer B.Cu) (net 4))
 (segment (start 13.25 25.25) (end 11.25 25.25) (width 1) (layer F.Cu) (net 4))
 (segment (start 14.028709 16.399999) (end 14.028709 16.471291) (width 1) (layer F.Cu) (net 4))
 (segment (start 11.25 25.25) (end 10 24) (width 1) (layer F.Cu) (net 4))
 (segment (start 14 24.5) (end 13.25 25.25) (width 1) (layer F.Cu) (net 4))
 (segment (start 13.62871 16) (end 14.028709 16.399999) (width 1) (layer F.Cu) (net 4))
 (segment (start 14.028709 16.471291) (end 14 16.5) (width 1) (layer F.Cu) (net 4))
 (segment (start 14 16.5) (end 14 24.5) (width 1) (layer F.Cu) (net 4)))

